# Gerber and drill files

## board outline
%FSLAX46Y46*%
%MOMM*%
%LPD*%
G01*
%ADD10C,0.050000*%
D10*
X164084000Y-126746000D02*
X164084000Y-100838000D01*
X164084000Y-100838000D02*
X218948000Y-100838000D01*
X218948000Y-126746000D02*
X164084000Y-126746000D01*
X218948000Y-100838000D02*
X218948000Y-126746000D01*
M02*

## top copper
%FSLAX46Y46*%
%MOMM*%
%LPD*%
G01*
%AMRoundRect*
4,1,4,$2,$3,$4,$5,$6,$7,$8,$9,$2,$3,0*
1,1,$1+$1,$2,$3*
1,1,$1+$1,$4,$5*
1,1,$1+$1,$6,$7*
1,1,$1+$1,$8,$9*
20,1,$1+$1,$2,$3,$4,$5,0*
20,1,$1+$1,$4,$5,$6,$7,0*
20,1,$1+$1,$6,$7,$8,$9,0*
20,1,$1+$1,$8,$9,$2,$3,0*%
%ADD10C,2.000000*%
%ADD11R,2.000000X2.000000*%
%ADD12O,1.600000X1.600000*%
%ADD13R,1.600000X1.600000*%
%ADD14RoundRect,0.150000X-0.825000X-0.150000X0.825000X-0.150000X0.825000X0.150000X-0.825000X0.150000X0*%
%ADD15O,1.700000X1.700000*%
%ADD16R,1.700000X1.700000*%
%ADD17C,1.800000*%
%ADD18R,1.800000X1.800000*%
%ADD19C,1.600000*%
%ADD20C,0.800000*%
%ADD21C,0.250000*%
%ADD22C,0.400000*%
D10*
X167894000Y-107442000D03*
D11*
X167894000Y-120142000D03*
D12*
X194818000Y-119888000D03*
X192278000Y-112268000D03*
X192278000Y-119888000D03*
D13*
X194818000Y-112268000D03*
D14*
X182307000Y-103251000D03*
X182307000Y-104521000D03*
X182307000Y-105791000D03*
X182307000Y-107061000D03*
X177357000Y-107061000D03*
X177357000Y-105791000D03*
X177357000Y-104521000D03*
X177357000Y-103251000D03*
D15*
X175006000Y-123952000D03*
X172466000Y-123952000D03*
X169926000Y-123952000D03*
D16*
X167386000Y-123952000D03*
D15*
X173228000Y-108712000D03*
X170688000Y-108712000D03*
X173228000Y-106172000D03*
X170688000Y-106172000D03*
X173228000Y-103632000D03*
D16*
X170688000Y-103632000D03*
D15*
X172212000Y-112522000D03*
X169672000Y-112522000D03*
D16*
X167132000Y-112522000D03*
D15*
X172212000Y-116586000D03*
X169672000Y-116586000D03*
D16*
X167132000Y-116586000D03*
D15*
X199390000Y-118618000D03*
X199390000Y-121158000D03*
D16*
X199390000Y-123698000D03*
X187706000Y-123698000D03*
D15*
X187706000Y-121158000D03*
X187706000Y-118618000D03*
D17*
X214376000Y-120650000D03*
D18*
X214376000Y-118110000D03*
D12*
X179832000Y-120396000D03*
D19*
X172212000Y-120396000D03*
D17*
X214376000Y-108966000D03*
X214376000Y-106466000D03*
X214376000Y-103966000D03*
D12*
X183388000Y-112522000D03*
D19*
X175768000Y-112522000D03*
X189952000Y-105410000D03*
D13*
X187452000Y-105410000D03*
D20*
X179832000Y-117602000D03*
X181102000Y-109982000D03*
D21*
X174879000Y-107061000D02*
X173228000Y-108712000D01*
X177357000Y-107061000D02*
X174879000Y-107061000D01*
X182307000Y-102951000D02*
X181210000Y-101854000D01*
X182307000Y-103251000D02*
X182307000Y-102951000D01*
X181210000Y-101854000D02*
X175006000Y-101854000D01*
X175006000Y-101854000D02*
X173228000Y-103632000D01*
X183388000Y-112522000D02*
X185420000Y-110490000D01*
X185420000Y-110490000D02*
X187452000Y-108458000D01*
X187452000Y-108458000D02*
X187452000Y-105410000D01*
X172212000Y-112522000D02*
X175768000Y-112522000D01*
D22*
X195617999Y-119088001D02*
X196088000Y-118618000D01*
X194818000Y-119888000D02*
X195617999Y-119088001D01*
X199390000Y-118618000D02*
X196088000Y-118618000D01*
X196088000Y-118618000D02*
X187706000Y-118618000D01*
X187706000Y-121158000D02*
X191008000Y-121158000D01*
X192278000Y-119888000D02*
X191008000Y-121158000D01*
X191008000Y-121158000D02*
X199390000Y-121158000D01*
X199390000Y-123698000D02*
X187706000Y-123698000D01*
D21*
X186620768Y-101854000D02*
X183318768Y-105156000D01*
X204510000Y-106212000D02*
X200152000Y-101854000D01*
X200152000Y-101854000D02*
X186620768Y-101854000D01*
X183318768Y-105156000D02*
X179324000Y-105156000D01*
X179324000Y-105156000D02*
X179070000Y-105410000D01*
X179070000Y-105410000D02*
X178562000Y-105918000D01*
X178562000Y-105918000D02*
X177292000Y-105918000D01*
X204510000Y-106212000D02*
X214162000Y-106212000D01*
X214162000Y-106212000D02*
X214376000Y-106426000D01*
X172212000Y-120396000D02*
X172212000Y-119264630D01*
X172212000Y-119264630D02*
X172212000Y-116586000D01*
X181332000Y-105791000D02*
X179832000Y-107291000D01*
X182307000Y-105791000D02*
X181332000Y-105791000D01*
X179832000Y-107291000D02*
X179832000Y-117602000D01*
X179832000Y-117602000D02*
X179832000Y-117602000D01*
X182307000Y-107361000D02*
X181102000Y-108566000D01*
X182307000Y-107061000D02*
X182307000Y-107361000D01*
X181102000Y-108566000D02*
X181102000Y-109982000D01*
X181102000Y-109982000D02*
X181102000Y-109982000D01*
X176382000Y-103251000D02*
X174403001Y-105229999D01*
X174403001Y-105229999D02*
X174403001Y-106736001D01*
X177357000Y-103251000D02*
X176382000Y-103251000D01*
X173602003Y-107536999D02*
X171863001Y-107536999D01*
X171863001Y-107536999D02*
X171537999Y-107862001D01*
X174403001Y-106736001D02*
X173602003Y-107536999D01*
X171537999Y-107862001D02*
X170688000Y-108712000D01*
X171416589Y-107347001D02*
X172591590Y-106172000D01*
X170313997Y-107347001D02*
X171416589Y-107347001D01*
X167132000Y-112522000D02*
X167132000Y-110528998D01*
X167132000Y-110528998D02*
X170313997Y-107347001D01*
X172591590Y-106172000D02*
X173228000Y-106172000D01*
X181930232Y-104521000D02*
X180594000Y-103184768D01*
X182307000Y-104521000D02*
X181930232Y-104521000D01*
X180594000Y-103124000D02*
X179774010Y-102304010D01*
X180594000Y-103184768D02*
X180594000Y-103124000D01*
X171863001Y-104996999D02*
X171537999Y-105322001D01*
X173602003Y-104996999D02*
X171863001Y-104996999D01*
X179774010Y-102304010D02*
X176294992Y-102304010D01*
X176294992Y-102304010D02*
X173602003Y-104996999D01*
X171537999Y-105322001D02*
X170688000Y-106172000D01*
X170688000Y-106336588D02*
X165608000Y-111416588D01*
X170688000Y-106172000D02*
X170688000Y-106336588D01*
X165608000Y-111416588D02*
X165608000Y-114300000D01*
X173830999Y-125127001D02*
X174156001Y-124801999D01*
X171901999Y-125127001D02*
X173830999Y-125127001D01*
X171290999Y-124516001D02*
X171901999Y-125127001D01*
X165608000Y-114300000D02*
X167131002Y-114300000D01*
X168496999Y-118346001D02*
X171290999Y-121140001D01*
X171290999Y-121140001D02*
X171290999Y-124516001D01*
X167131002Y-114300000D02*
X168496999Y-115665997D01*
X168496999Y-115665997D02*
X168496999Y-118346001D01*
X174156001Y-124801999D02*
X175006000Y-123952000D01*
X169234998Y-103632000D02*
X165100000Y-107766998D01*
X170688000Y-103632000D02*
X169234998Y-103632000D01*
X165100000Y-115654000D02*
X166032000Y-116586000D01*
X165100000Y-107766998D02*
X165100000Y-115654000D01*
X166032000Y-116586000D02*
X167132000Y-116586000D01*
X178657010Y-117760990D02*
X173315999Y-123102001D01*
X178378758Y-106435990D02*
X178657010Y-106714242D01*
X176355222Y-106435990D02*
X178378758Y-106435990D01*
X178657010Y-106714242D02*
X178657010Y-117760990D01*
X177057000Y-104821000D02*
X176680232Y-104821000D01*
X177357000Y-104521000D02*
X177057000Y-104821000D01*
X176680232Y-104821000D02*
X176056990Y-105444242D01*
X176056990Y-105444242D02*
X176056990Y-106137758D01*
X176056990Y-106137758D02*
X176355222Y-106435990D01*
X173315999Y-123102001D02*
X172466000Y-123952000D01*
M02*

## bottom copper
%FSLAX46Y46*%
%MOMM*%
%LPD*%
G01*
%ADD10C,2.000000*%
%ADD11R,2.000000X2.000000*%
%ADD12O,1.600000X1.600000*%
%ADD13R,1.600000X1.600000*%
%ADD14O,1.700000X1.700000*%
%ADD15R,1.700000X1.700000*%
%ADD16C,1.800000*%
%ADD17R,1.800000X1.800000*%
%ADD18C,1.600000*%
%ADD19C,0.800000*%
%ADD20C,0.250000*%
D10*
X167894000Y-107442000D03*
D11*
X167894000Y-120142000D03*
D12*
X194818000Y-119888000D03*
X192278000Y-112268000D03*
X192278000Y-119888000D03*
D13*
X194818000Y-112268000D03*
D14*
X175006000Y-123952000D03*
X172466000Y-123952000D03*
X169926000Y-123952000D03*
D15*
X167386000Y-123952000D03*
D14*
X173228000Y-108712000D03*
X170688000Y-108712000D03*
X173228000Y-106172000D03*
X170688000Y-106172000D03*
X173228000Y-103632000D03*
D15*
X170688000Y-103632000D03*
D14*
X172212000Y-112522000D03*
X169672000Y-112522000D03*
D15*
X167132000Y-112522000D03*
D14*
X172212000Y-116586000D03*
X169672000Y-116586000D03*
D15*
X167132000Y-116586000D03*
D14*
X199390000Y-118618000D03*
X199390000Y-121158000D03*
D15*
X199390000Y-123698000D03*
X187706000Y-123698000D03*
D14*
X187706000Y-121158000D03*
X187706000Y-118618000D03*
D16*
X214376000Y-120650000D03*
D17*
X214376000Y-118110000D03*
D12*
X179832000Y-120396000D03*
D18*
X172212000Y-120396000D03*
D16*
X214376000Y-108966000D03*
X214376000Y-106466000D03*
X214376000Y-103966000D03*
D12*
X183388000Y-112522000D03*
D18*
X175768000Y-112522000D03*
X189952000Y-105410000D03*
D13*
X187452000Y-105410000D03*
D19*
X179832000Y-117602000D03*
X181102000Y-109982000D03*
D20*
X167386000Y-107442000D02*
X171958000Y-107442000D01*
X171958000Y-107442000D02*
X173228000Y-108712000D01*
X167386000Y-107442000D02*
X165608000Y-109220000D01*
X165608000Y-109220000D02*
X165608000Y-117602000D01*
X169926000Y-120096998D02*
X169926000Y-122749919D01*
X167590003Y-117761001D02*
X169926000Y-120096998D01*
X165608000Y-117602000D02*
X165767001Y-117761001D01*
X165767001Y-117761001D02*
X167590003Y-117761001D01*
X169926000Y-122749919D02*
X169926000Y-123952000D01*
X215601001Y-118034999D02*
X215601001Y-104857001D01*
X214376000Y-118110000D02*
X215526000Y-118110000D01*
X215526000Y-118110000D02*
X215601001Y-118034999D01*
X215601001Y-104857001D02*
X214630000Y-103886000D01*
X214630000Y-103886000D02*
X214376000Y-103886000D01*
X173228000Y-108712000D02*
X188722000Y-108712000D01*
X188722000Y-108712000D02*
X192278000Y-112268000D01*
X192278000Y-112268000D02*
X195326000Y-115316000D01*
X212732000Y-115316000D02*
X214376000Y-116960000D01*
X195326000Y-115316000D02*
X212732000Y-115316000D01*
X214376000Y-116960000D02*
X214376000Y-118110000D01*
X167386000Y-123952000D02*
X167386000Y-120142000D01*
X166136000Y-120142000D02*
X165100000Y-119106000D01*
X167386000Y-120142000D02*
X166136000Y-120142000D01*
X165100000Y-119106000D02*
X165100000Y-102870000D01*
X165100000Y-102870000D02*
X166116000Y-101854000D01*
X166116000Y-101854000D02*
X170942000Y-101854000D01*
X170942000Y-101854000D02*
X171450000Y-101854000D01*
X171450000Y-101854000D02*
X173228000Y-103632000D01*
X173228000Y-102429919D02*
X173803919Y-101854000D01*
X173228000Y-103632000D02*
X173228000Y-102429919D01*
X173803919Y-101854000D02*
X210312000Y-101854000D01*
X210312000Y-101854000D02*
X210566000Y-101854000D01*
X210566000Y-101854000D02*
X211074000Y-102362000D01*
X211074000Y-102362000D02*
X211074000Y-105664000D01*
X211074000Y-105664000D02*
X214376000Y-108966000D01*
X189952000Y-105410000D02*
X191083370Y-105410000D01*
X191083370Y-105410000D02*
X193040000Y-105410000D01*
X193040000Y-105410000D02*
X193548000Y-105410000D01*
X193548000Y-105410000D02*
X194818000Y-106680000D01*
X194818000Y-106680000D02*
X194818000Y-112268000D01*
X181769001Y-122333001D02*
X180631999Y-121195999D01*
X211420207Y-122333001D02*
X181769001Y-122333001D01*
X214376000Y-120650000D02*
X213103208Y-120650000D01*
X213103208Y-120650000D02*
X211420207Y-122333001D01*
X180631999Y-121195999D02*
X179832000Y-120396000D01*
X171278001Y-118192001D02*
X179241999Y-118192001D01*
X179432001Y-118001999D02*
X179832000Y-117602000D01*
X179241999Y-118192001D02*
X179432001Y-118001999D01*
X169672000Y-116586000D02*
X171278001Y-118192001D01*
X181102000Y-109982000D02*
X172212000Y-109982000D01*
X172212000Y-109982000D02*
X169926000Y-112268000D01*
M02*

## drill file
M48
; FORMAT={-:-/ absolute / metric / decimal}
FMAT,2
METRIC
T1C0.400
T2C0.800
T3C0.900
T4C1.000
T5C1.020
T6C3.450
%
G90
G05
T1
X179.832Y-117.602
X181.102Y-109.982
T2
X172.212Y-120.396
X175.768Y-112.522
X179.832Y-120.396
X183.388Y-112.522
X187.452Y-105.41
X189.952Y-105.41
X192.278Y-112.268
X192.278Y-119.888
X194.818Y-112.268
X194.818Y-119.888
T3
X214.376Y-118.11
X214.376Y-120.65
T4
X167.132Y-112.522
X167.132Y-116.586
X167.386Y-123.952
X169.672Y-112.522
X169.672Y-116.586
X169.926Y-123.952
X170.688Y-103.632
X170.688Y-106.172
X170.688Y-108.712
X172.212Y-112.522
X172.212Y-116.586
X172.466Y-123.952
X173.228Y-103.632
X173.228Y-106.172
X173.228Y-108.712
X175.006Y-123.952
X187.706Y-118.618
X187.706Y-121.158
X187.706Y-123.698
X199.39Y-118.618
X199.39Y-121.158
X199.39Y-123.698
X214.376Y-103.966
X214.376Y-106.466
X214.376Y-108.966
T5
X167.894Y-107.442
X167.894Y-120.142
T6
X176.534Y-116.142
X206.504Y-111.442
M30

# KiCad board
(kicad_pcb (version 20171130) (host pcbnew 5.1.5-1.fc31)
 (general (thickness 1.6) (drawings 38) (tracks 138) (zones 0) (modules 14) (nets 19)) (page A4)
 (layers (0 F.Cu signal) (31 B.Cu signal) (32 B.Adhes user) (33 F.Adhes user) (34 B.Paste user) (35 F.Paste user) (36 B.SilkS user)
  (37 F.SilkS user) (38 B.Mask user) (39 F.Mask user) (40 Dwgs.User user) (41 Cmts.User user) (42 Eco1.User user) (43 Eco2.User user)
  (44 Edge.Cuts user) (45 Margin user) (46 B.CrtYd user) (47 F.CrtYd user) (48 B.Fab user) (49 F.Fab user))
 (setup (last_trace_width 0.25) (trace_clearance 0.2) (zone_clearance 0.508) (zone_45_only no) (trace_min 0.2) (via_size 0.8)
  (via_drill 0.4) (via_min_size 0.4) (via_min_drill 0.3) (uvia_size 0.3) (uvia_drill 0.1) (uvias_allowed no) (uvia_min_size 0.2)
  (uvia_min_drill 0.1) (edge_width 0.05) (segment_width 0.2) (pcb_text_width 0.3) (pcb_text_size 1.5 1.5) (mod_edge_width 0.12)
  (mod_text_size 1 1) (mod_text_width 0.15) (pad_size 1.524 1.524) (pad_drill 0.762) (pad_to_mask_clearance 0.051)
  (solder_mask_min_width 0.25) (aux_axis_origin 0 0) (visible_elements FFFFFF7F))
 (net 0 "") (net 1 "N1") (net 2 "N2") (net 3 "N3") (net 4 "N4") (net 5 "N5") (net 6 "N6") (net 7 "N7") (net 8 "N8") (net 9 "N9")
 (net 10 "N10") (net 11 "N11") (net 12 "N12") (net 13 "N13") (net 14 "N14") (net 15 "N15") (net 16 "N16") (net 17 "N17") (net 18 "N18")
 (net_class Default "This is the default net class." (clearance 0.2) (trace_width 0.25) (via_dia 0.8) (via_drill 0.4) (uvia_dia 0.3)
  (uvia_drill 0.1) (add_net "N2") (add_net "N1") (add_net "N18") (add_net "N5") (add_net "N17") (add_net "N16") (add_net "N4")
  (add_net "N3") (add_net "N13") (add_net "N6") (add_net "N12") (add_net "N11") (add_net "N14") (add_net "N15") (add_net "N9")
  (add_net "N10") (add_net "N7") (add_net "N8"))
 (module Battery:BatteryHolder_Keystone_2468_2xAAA (layer B.Cu) (at 167.894 120.142)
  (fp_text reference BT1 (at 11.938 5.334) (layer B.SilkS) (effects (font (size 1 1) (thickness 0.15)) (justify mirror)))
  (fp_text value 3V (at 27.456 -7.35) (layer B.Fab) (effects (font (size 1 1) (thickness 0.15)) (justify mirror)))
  (pad "" np_thru_hole circle (at 38.61 -8.7) (size 3.45 3.45) (drill 3.45) (layers *.Cu *.Mask))
  (pad "" np_thru_hole circle (at 8.64 -4) (size 3.45 3.45) (drill 3.45) (layers *.Cu))
  (pad 2 thru_hole circle (at 0 -12.7) (size 2 2) (drill 1.02) (layers *.Cu *.Mask) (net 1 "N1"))
  (pad 1 thru_hole rect (at 0 0) (size 2 2) (drill 1.02) (layers *.Cu *.Mask) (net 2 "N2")))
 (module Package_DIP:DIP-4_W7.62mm (layer F.Cu) (at 194.818 112.268 270)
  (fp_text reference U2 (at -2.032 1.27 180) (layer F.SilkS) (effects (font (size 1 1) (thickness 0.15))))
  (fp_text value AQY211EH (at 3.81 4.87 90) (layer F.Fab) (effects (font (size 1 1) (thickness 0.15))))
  (pad 4 thru_hole oval (at 7.62 0 270) (size 1.6 1.6) (drill 0.8) (layers *.Cu *.Mask) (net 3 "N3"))
  (pad 2 thru_hole oval (at 0 2.54 270) (size 1.6 1.6) (drill 0.8) (layers *.Cu *.Mask) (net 1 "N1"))
  (pad 3 thru_hole oval (at 7.62 2.54 270) (size 1.6 1.6) (drill 0.8) (layers *.Cu *.Mask) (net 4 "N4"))
  (pad 1 thru_hole rect (at 0 0 270) (size 1.6 1.6) (drill 0.8) (layers *.Cu *.Mask) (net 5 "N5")))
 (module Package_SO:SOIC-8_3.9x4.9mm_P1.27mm (layer F.Cu) (at 179.832 105.156)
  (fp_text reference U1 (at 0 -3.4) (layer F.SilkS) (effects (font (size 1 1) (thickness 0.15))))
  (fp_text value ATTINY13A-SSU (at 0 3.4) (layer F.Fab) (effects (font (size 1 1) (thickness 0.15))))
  (pad 8 smd roundrect (at 2.475 -1.905) (size 1.95 0.6) (layers F.Cu F.Paste F.Mask) (roundrect_rratio 0.25) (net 2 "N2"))
  (pad 7 smd roundrect (at 2.475 -0.635) (size 1.95 0.6) (layers F.Cu F.Paste F.Mask) (roundrect_rratio 0.25) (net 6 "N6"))
  (pad 6 smd roundrect (at 2.475 0.635) (size 1.95 0.6) (layers F.Cu F.Paste F.Mask) (roundrect_rratio 0.25) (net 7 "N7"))
  (pad 5 smd roundrect (at 2.475 1.905) (size 1.95 0.6) (layers F.Cu F.Paste F.Mask) (roundrect_rratio 0.25) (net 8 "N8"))
  (pad 4 smd roundrect (at -2.475 1.905) (size 1.95 0.6) (layers F.Cu F.Paste F.Mask) (roundrect_rratio 0.25) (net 1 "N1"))
  (pad 3 smd roundrect (at -2.475 0.635) (size 1.95 0.6) (layers F.Cu F.Paste F.Mask) (roundrect_rratio 0.25) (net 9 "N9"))
  (pad 2 smd roundrect (at -2.475 -0.635) (size 1.95 0.6) (layers F.Cu F.Paste F.Mask) (roundrect_rratio 0.25) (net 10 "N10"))
  (pad 1 smd roundrect (at -2.475 -1.905) (size 1.95 0.6) (layers F.Cu F.Paste F.Mask) (roundrect_rratio 0.25) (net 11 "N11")))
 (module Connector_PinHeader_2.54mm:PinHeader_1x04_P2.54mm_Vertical (layer F.Cu) (at 167.386 123.952 90)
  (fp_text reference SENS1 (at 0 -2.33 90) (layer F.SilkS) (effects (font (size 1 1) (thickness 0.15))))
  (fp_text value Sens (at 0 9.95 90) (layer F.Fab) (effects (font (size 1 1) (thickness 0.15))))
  (pad 4 thru_hole oval (at 0 7.62 90) (size 1.7 1.7) (drill 1) (layers *.Cu *.Mask) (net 6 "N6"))
  (pad 3 thru_hole oval (at 0 5.08 90) (size 1.7 1.7) (drill 1) (layers *.Cu *.Mask) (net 10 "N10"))
  (pad 2 thru_hole oval (at 0 2.54 90) (size 1.7 1.7) (drill 1) (layers *.Cu *.Mask) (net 1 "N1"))
  (pad 1 thru_hole rect (at 0 0 90) (size 1.7 1.7) (drill 1) (layers *.Cu *.Mask) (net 2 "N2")))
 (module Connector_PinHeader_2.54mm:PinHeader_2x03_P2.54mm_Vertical (layer F.Cu) (at 170.688 103.632)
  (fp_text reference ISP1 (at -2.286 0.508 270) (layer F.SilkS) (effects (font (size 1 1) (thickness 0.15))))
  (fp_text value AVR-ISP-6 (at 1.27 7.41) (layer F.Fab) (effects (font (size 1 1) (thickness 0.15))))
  (pad 6 thru_hole oval (at 2.54 5.08) (size 1.7 1.7) (drill 1) (layers *.Cu *.Mask) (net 1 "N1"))
  (pad 5 thru_hole oval (at 0 5.08) (size 1.7 1.7) (drill 1) (layers *.Cu *.Mask) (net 11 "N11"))
  (pad 4 thru_hole oval (at 2.54 2.54) (size 1.7 1.7) (drill 1) (layers *.Cu *.Mask) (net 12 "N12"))
  (pad 3 thru_hole oval (at 0 2.54) (size 1.7 1.7) (drill 1) (layers *.Cu *.Mask) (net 6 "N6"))
  (pad 2 thru_hole oval (at 2.54 0) (size 1.7 1.7) (drill 1) (layers *.Cu *.Mask) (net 2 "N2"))
  (pad 1 thru_hole rect (at 0 0) (size 1.7 1.7) (drill 1) (layers *.Cu *.Mask) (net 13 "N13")))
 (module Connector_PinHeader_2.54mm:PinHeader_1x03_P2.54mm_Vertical (layer F.Cu) (at 167.132 112.522 90)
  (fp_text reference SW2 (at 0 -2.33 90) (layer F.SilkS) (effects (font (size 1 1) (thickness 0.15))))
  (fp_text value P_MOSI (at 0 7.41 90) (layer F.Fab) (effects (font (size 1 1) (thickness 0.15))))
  (pad 3 thru_hole oval (at 0 5.08 90) (size 1.7 1.7) (drill 1) (layers *.Cu *.Mask) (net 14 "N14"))
  (pad 2 thru_hole oval (at 0 2.54 90) (size 1.7 1.7) (drill 1) (layers *.Cu *.Mask) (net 8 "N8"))
  (pad 1 thru_hole rect (at 0 0 90) (size 1.7 1.7) (drill 1) (layers *.Cu *.Mask) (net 12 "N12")))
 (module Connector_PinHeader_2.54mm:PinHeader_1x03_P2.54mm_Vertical (layer F.Cu) (at 167.132 116.586 90)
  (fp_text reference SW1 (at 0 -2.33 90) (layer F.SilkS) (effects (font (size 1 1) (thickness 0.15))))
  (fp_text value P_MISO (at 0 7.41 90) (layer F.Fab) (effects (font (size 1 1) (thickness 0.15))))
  (pad 3 thru_hole oval (at 0 5.08 90) (size 1.7 1.7) (drill 1) (layers *.Cu *.Mask) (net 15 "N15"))
  (pad 2 thru_hole oval (at 0 2.54 90) (size 1.7 1.7) (drill 1) (layers *.Cu *.Mask) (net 7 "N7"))
  (pad 1 thru_hole rect (at 0 0 90) (size 1.7 1.7) (drill 1) (layers *.Cu *.Mask) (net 13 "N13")))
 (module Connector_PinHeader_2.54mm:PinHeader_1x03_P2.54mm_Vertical (layer F.Cu) (at 199.39 123.698 180)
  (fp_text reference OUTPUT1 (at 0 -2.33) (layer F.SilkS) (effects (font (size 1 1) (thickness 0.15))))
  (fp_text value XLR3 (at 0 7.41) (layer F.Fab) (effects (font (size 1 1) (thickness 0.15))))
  (pad 3 thru_hole oval (at 0 5.08 180) (size 1.7 1.7) (drill 1) (layers *.Cu *.Mask) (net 3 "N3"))
  (pad 2 thru_hole oval (at 0 2.54 180) (size 1.7 1.7) (drill 1) (layers *.Cu *.Mask) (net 4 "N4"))
  (pad 1 thru_hole rect (at 0 0 180) (size 1.7 1.7) (drill 1) (layers *.Cu *.Mask) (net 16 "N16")))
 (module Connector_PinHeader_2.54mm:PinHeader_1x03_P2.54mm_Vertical (layer F.Cu) (at 187.706 123.698 180)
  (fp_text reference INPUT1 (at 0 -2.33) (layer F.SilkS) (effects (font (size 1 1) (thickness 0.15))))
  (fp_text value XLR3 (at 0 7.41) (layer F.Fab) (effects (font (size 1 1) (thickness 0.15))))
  (pad 1 thru_hole rect (at 0 0 180) (size 1.7 1.7) (drill 1) (layers *.Cu *.Mask) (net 16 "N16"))
  (pad 2 thru_hole oval (at 0 2.54 180) (size 1.7 1.7) (drill 1) (layers *.Cu *.Mask) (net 4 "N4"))
  (pad 3 thru_hole oval (at 0 5.08 180) (size 1.7 1.7) (drill 1) (layers *.Cu *.Mask) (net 3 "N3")))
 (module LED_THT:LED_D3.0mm (layer F.Cu) (at 214.376 118.11 270)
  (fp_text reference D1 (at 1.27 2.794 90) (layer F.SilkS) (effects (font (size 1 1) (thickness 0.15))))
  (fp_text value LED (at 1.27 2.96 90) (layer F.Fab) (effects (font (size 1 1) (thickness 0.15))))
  (pad 2 thru_hole circle (at 2.54 0 270) (size 1.8 1.8) (drill 0.9) (layers *.Cu *.Mask) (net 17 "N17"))
  (pad 1 thru_hole rect (at 0 0 270) (size 1.8 1.8) (drill 0.9) (layers *.Cu *.Mask) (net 1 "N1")))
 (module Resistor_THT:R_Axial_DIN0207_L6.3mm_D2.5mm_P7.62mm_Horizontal (layer F.Cu) (at 172.212 120.396)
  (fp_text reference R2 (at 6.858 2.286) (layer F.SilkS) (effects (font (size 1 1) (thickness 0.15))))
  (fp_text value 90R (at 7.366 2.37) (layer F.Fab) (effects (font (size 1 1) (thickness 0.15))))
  (pad 2 thru_hole oval (at 7.62 0) (size 1.6 1.6) (drill 0.8) (layers *.Cu *.Mask) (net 17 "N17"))
  (pad 1 thru_hole circle (at 0 0) (size 1.6 1.6) (drill 0.8) (layers *.Cu *.Mask) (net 15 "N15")))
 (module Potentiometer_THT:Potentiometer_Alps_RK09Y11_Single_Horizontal (layer F.Cu) (at 214.376 108.966)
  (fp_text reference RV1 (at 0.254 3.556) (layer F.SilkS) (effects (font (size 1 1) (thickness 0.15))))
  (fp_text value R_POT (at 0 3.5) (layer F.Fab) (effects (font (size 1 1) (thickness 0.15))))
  (pad 1 thru_hole circle (at 0 0) (size 1.8 1.8) (drill 1) (layers *.Cu *.Mask) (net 2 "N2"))
  (pad 2 thru_hole circle (at 0 -2.5) (size 1.8 1.8) (drill 1) (layers *.Cu *.Mask) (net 9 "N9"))
  (pad 3 thru_hole circle (at 0 -5) (size 1.8 1.8) (drill 1) (layers *.Cu *.Mask) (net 1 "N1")))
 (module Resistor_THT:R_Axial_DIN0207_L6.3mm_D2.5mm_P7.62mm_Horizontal (layer F.Cu) (at 175.768 112.522)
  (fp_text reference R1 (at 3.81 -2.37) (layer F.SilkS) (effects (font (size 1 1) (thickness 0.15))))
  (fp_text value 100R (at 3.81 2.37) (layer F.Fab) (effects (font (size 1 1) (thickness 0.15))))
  (pad 2 thru_hole oval (at 7.62 0) (size 1.6 1.6) (drill 0.8) (layers *.Cu *.Mask) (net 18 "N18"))
  (pad 1 thru_hole circle (at 0 0) (size 1.6 1.6) (drill 0.8) (layers *.Cu *.Mask) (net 14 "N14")))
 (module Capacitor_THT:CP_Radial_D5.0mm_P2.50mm (layer F.Cu) (at 187.452 105.41)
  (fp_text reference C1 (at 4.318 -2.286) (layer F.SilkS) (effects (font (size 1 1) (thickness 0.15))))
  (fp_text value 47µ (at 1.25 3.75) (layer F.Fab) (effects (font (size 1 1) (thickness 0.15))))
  (pad 2 thru_hole circle (at 2.5 0) (size 1.6 1.6) (drill 0.8) (layers *.Cu *.Mask) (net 5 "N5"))
  (pad 1 thru_hole rect (at 0 0) (size 1.6 1.6) (drill 0.8) (layers *.Cu *.Mask) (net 18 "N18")))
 (gr_line (start 164.084 126.746) (end 164.084 100.838) (layer Edge.Cuts) (width 0.05))
 (gr_line (start 164.084 100.838) (end 218.948 100.838) (layer Edge.Cuts) (width 0.05))
 (gr_line (start 218.948 126.746) (end 164.084 126.746) (layer Edge.Cuts) (width 0.05))
 (gr_line (start 218.948 100.838) (end 218.948 126.746) (layer Edge.Cuts) (width 0.05))
 (segment (start 174.879 107.061) (end 173.228 108.712) (width 0.25) (layer F.Cu) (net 1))
 (segment (start 177.357 107.061) (end 174.879 107.061) (width 0.25) (layer F.Cu) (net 1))
 (segment (start 167.386 107.442) (end 171.958 107.442) (width 0.25) (layer B.Cu) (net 1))
 (segment (start 171.958 107.442) (end 173.228 108.712) (width 0.25) (layer B.Cu) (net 1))
 (segment (start 167.386 107.442) (end 165.608 109.22) (width 0.25) (layer B.Cu) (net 1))
 (segment (start 165.608 109.22) (end 165.608 117.602) (width 0.25) (layer B.Cu) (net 1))
 (segment (start 169.926 120.096998) (end 169.926 122.749919) (width 0.25) (layer B.Cu) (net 1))
 (segment (start 167.590003 117.761001) (end 169.926 120.096998) (width 0.25) (layer B.Cu) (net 1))
 (segment (start 165.608 117.602) (end 165.767001 117.761001) (width 0.25) (layer B.Cu) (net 1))
 (segment (start 165.767001 117.761001) (end 167.590003 117.761001) (width 0.25) (layer B.Cu) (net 1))
 (segment (start 169.926 122.749919) (end 169.926 123.952) (width 0.25) (layer B.Cu) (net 1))
 (segment (start 215.601001 118.034999) (end 215.601001 104.857001) (width 0.25) (layer B.Cu) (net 1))
 (segment (start 214.376 118.11) (end 215.526 118.11) (width 0.25) (layer B.Cu) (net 1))
 (segment (start 215.526 118.11) (end 215.601001 118.034999) (width 0.25) (layer B.Cu) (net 1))
 (segment (start 215.601001 104.857001) (end 214.63 103.886) (width 0.25) (layer B.Cu) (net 1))
 (segment (start 214.63 103.886) (end 214.376 103.886) (width 0.25) (layer B.Cu) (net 1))
 (segment (start 173.228 108.712) (end 188.722 108.712) (width 0.25) (layer B.Cu) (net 1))
 (segment (start 188.722 108.712) (end 192.278 112.268) (width 0.25) (layer B.Cu) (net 1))
 (segment (start 192.278 112.268) (end 195.326 115.316) (width 0.25) (layer B.Cu) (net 1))
 (segment (start 212.732 115.316) (end 214.376 116.96) (width 0.25) (layer B.Cu) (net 1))
 (segment (start 195.326 115.316) (end 212.732 115.316) (width 0.25) (layer B.Cu) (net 1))
 (segment (start 214.376 116.96) (end 214.376 118.11) (width 0.25) (layer B.Cu) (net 1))
 (segment (start 167.386 123.952) (end 167.386 120.142) (width 0.25) (layer B.Cu) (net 2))
 (segment (start 166.136 120.142) (end 165.1 119.106) (width 0.25) (layer B.Cu) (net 2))
 (segment (start 167.386 120.142) (end 166.136 120.142) (width 0.25) (layer B.Cu) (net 2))
 (segment (start 165.1 119.106) (end 165.1 102.87) (width 0.25) (layer B.Cu) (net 2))
 (segment (start 165.1 102.87) (end 166.116 101.854) (width 0.25) (layer B.Cu) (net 2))
 (segment (start 166.116 101.854) (end 170.942 101.854) (width 0.25) (layer B.Cu) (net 2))
 (segment (start 170.942 101.854) (end 171.45 101.854) (width 0.25) (layer B.Cu) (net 2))
 (segment (start 171.45 101.854) (end 173.228 103.632) (width 0.25) (layer B.Cu) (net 2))
 (segment (start 173.228 102.429919) (end 173.803919 101.854) (width 0.25) (layer B.Cu) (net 2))
 (segment (start 173.228 103.632) (end 173.228 102.429919) (width 0.25) (layer B.Cu) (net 2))
 (segment (start 173.803919 101.854) (end 210.312 101.854) (width 0.25) (layer B.Cu) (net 2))
 (segment (start 182.307 102.951) (end 181.21 101.854) (width 0.25) (layer F.Cu) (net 2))
 (segment (start 182.307 103.251) (end 182.307 102.951) (width 0.25) (layer F.Cu) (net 2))
 (segment (start 181.21 101.854) (end 175.006 101.854) (width 0.25) (layer F.Cu) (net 2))
 (segment (start 175.006 101.854) (end 173.228 103.632) (width 0.25) (layer F.Cu) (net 2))
 (segment (start 210.312 101.854) (end 210.566 101.854) (width 0.25) (layer B.Cu) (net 2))
 (segment (start 210.566 101.854) (end 211.074 102.362) (width 0.25) (layer B.Cu) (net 2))
 (segment (start 211.074 102.362) (end 211.074 105.664) (width 0.25) (layer B.Cu) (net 2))
 (segment (start 211.074 105.664) (end 214.376 108.966) (width 0.25) (layer B.Cu) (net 2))
 (segment (start 189.952 105.41) (end 191.08337 105.41) (width 0.25) (layer B.Cu) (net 5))
 (segment (start 191.08337 105.41) (end 193.04 105.41) (width 0.25) (layer B.Cu) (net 5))
 (segment (start 193.04 105.41) (end 193.548 105.41) (width 0.25) (layer B.Cu) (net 5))
 (segment (start 193.548 105.41) (end 194.818 106.68) (width 0.25) (layer B.Cu) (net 5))
 (segment (start 194.818 106.68) (end 194.818 112.268) (width 0.25) (layer B.Cu) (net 5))
 (segment (start 183.388 112.522) (end 185.42 110.49) (width 0.25) (layer F.Cu) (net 18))
 (segment (start 185.42 110.49) (end 187.452 108.458) (width 0.25) (layer F.Cu) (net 18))
 (segment (start 187.452 108.458) (end 187.452 105.41) (width 0.25) (layer F.Cu) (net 18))
 (segment (start 172.212 112.522) (end 175.768 112.522) (width 0.25) (layer F.Cu) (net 14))
 (segment (start 195.617999 119.088001) (end 196.088 118.618) (width 0.4) (layer F.Cu) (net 3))
 (segment (start 194.818 119.888) (end 195.617999 119.088001) (width 0.4) (layer F.Cu) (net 3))
 (segment (start 199.39 118.618) (end 196.088 118.618) (width 0.4) (layer F.Cu) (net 3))
 (segment (start 196.088 118.618) (end 187.706 118.618) (width 0.4) (layer F.Cu) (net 3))
 (segment (start 187.706 121.158) (end 191.008 121.158) (width 0.4) (layer F.Cu) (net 4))
 (segment (start 192.278 119.888) (end 191.008 121.158) (width 0.4) (layer F.Cu) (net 4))
 (segment (start 191.008 121.158) (end 199.39 121.158) (width 0.4) (layer F.Cu) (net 4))
 (segment (start 199.39 123.698) (end 187.706 123.698) (width 0.4) (layer F.Cu) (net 16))
 (segment (start 186.620768 101.854) (end 183.318768 105.156) (width 0.25) (layer F.Cu) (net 9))
 (segment (start 204.51 106.212) (end 200.152 101.854) (width 0.25) (layer F.Cu) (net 9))
 (segment (start 200.152 101.854) (end 186.620768 101.854) (width 0.25) (layer F.Cu) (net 9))
 (segment (start 183.318768 105.156) (end 179.324 105.156) (width 0.25) (layer F.Cu) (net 9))
 (segment (start 179.324 105.156) (end 179.07 105.41) (width 0.25) (layer F.Cu) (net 9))
 (segment (start 179.07 105.41) (end 178.562 105.918) (width 0.25) (layer F.Cu) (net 9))
 (segment (start 178.562 105.918) (end 177.292 105.918) (width 0.25) (layer F.Cu) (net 9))
 (segment (start 204.51 106.212) (end 214.162 106.212) (width 0.25) (layer F.Cu) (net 9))
 (segment (start 214.162 106.212) (end 214.376 106.426) (width 0.25) (layer F.Cu) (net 9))
 (segment (start 181.769001 122.333001) (end 180.631999 121.195999) (width 0.25) (layer B.Cu) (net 17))
 (segment (start 211.420207 122.333001) (end 181.769001 122.333001) (width 0.25) (layer B.Cu) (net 17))
 (segment (start 214.376 120.65) (end 213.103208 120.65) (width 0.25) (layer B.Cu) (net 17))
 (segment (start 213.103208 120.65) (end 211.420207 122.333001) (width 0.25) (layer B.Cu) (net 17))
 (segment (start 180.631999 121.195999) (end 179.832 120.396) (width 0.25) (layer B.Cu) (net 17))
 (segment (start 172.212 120.396) (end 172.212 119.26463) (width 0.25) (layer F.Cu) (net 15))
 (segment (start 172.212 119.26463) (end 172.212 116.586) (width 0.25) (layer F.Cu) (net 15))
 (segment (start 181.332 105.791) (end 179.832 107.291) (width 0.25) (layer F.Cu) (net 7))
 (segment (start 182.307 105.791) (end 181.332 105.791) (width 0.25) (layer F.Cu) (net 7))
 (segment (start 179.832 107.291) (end 179.832 117.602) (width 0.25) (layer F.Cu) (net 7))
 (segment (start 179.832 117.602) (end 179.832 117.602) (width 0.25) (layer F.Cu) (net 7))
 (via (at 179.832 117.602) (size 0.8) (drill 0.4) (layers F.Cu B.Cu) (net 7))
 (segment (start 171.278001 118.192001) (end 179.241999 118.192001) (width 0.25) (layer B.Cu) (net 7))
 (segment (start 179.432001 118.001999) (end 179.832 117.602) (width 0.25) (layer B.Cu) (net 7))
 (segment (start 179.241999 118.192001) (end 179.432001 118.001999) (width 0.25) (layer B.Cu) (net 7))
 (segment (start 169.672 116.586) (end 171.278001 118.192001) (width 0.25) (layer B.Cu) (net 7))
 (segment (start 182.307 107.361) (end 181.102 108.566) (width 0.25) (layer F.Cu) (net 8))
 (segment (start 182.307 107.061) (end 182.307 107.361) (width 0.25) (layer F.Cu) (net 8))
 (segment (start 181.102 108.566) (end 181.102 109.982) (width 0.25) (layer F.Cu) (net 8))
 (segment (start 181.102 109.982) (end 181.102 109.982) (width 0.25) (layer F.Cu) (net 8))
 (via (at 181.102 109.982) (size 0.8) (drill 0.4) (layers F.Cu B.Cu) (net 8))
 (segment (start 181.102 109.982) (end 172.212 109.982) (width 0.25) (layer B.Cu) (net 8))
 (segment (start 172.212 109.982) (end 169.926 112.268) (width 0.25) (layer B.Cu) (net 8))
 (segment (start 176.382 103.251) (end 174.403001 105.229999) (width 0.25) (layer F.Cu) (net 11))
 (segment (start 174.403001 105.229999) (end 174.403001 106.736001) (width 0.25) (layer F.Cu) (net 11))
 (segment (start 177.357 103.251) (end 176.382 103.251) (width 0.25) (layer F.Cu) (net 11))
 (segment (start 173.602003 107.536999) (end 171.863001 107.536999) (width 0.25) (layer F.Cu) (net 11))
 (segment (start 171.863001 107.536999) (end 171.537999 107.862001) (width 0.25) (layer F.Cu) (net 11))
 (segment (start 174.403001 106.736001) (end 173.602003 107.536999) (width 0.25) (layer F.Cu) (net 11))
 (segment (start 171.537999 107.862001) (end 170.688 108.712) (width 0.25) (layer F.Cu) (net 11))
 (segment (start 171.416589 107.347001) (end 172.59159 106.172) (width 0.25) (layer F.Cu) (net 12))
 (segment (start 170.313997 107.347001) (end 171.416589 107.347001) (width 0.25) (layer F.Cu) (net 12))
 (segment (start 167.132 112.522) (end 167.132 110.528998) (width 0.25) (layer F.Cu) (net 12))
 (segment (start 167.132 110.528998) (end 170.313997 107.347001) (width 0.25) (layer F.Cu) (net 12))
 (segment (start 172.59159 106.172) (end 173.228 106.172) (width 0.25) (layer F.Cu) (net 12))
 (segment (start 181.930232 104.521) (end 180.594 103.184768) (width 0.25) (layer F.Cu) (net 6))
 (segment (start 182.307 104.521) (end 181.930232 104.521) (width 0.25) (layer F.Cu) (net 6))
 (segment (start 180.594 103.124) (end 179.77401 102.30401) (width 0.25) (layer F.Cu) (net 6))
 (segment (start 180.594 103.184768) (end 180.594 103.124) (width 0.25) (layer F.Cu) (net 6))
 (segment (start 171.863001 104.996999) (end 171.537999 105.322001) (width 0.25) (layer F.Cu) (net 6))
 (segment (start 173.602003 104.996999) (end 171.863001 104.996999) (width 0.25) (layer F.Cu) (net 6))
 (segment (start 179.77401 102.30401) (end 176.294992 102.30401) (width 0.25) (layer F.Cu) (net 6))
 (segment (start 176.294992 102.30401) (end 173.602003 104.996999) (width 0.25) (layer F.Cu) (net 6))
 (segment (start 171.537999 105.322001) (end 170.688 106.172) (width 0.25) (layer F.Cu) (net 6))
 (segment (start 170.688 106.336588) (end 165.608 111.416588) (width 0.25) (layer F.Cu) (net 6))
 (segment (start 170.688 106.172) (end 170.688 106.336588) (width 0.25) (layer F.Cu) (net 6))
 (segment (start 165.608 111.416588) (end 165.608 114.3) (width 0.25) (layer F.Cu) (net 6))
 (segment (start 173.830999 125.127001) (end 174.156001 124.801999) (width 0.25) (layer F.Cu) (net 6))
 (segment (start 171.901999 125.127001) (end 173.830999 125.127001) (width 0.25) (layer F.Cu) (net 6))
 (segment (start 171.290999 124.516001) (end 171.901999 125.127001) (width 0.25) (layer F.Cu) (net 6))
 (segment (start 165.608 114.3) (end 167.131002 114.3) (width 0.25) (layer F.Cu) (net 6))
 (segment (start 168.496999 118.346001) (end 171.290999 121.140001) (width 0.25) (layer F.Cu) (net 6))
 (segment (start 171.290999 121.140001) (end 171.290999 124.516001) (width 0.25) (layer F.Cu) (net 6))
 (segment (start 167.131002 114.3) (end 168.496999 115.665997) (width 0.25) (layer F.Cu) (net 6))
 (segment (start 168.496999 115.665997) (end 168.496999 118.346001) (width 0.25) (layer F.Cu) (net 6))
 (segment (start 174.156001 124.801999) (end 175.006 123.952) (width 0.25) (layer F.Cu) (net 6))
 (segment (start 169.234998 103.632) (end 165.1 107.766998) (width 0.25) (layer F.Cu) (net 13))
 (segment (start 170.688 103.632) (end 169.234998 103.632) (width 0.25) (layer F.Cu) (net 13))
 (segment (start 165.1 115.654) (end 166.032 116.586) (width 0.25) (layer F.Cu) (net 13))
 (segment (start 165.1 107.766998) (end 165.1 115.654) (width 0.25) (layer F.Cu) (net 13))
 (segment (start 166.032 116.586) (end 167.132 116.586) (width 0.25) (layer F.Cu) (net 13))
 (segment (start 178.65701 117.76099) (end 173.315999 123.102001) (width 0.25) (layer F.Cu) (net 10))
 (segment (start 178.378758 106.43599) (end 178.65701 106.714242) (width 0.25) (layer F.Cu) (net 10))
 (segment (start 176.355222 106.43599) (end 178.378758 106.43599) (width 0.25) (layer F.Cu) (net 10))
 (segment (start 178.65701 106.714242) (end 178.65701 117.76099) (width 0.25) (layer F.Cu) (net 10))
 (segment (start 177.057 104.821) (end 176.680232 104.821) (width 0.25) (layer F.Cu) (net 10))
 (segment (start 177.357 104.521) (end 177.057 104.821) (width 0.25) (layer F.Cu) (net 10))
 (segment (start 176.680232 104.821) (end 176.05699 105.444242) (width 0.25) (layer F.Cu) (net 10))
 (segment (start 176.05699 105.444242) (end 176.05699 106.137758) (width 0.25) (layer F.Cu) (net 10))
 (segment (start 176.05699 106.137758) (end 176.355222 106.43599) (width 0.25) (layer F.Cu) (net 10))
 (segment (start 173.315999 123.102001) (end 172.466 123.952) (width 0.25) (layer F.Cu) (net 10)))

